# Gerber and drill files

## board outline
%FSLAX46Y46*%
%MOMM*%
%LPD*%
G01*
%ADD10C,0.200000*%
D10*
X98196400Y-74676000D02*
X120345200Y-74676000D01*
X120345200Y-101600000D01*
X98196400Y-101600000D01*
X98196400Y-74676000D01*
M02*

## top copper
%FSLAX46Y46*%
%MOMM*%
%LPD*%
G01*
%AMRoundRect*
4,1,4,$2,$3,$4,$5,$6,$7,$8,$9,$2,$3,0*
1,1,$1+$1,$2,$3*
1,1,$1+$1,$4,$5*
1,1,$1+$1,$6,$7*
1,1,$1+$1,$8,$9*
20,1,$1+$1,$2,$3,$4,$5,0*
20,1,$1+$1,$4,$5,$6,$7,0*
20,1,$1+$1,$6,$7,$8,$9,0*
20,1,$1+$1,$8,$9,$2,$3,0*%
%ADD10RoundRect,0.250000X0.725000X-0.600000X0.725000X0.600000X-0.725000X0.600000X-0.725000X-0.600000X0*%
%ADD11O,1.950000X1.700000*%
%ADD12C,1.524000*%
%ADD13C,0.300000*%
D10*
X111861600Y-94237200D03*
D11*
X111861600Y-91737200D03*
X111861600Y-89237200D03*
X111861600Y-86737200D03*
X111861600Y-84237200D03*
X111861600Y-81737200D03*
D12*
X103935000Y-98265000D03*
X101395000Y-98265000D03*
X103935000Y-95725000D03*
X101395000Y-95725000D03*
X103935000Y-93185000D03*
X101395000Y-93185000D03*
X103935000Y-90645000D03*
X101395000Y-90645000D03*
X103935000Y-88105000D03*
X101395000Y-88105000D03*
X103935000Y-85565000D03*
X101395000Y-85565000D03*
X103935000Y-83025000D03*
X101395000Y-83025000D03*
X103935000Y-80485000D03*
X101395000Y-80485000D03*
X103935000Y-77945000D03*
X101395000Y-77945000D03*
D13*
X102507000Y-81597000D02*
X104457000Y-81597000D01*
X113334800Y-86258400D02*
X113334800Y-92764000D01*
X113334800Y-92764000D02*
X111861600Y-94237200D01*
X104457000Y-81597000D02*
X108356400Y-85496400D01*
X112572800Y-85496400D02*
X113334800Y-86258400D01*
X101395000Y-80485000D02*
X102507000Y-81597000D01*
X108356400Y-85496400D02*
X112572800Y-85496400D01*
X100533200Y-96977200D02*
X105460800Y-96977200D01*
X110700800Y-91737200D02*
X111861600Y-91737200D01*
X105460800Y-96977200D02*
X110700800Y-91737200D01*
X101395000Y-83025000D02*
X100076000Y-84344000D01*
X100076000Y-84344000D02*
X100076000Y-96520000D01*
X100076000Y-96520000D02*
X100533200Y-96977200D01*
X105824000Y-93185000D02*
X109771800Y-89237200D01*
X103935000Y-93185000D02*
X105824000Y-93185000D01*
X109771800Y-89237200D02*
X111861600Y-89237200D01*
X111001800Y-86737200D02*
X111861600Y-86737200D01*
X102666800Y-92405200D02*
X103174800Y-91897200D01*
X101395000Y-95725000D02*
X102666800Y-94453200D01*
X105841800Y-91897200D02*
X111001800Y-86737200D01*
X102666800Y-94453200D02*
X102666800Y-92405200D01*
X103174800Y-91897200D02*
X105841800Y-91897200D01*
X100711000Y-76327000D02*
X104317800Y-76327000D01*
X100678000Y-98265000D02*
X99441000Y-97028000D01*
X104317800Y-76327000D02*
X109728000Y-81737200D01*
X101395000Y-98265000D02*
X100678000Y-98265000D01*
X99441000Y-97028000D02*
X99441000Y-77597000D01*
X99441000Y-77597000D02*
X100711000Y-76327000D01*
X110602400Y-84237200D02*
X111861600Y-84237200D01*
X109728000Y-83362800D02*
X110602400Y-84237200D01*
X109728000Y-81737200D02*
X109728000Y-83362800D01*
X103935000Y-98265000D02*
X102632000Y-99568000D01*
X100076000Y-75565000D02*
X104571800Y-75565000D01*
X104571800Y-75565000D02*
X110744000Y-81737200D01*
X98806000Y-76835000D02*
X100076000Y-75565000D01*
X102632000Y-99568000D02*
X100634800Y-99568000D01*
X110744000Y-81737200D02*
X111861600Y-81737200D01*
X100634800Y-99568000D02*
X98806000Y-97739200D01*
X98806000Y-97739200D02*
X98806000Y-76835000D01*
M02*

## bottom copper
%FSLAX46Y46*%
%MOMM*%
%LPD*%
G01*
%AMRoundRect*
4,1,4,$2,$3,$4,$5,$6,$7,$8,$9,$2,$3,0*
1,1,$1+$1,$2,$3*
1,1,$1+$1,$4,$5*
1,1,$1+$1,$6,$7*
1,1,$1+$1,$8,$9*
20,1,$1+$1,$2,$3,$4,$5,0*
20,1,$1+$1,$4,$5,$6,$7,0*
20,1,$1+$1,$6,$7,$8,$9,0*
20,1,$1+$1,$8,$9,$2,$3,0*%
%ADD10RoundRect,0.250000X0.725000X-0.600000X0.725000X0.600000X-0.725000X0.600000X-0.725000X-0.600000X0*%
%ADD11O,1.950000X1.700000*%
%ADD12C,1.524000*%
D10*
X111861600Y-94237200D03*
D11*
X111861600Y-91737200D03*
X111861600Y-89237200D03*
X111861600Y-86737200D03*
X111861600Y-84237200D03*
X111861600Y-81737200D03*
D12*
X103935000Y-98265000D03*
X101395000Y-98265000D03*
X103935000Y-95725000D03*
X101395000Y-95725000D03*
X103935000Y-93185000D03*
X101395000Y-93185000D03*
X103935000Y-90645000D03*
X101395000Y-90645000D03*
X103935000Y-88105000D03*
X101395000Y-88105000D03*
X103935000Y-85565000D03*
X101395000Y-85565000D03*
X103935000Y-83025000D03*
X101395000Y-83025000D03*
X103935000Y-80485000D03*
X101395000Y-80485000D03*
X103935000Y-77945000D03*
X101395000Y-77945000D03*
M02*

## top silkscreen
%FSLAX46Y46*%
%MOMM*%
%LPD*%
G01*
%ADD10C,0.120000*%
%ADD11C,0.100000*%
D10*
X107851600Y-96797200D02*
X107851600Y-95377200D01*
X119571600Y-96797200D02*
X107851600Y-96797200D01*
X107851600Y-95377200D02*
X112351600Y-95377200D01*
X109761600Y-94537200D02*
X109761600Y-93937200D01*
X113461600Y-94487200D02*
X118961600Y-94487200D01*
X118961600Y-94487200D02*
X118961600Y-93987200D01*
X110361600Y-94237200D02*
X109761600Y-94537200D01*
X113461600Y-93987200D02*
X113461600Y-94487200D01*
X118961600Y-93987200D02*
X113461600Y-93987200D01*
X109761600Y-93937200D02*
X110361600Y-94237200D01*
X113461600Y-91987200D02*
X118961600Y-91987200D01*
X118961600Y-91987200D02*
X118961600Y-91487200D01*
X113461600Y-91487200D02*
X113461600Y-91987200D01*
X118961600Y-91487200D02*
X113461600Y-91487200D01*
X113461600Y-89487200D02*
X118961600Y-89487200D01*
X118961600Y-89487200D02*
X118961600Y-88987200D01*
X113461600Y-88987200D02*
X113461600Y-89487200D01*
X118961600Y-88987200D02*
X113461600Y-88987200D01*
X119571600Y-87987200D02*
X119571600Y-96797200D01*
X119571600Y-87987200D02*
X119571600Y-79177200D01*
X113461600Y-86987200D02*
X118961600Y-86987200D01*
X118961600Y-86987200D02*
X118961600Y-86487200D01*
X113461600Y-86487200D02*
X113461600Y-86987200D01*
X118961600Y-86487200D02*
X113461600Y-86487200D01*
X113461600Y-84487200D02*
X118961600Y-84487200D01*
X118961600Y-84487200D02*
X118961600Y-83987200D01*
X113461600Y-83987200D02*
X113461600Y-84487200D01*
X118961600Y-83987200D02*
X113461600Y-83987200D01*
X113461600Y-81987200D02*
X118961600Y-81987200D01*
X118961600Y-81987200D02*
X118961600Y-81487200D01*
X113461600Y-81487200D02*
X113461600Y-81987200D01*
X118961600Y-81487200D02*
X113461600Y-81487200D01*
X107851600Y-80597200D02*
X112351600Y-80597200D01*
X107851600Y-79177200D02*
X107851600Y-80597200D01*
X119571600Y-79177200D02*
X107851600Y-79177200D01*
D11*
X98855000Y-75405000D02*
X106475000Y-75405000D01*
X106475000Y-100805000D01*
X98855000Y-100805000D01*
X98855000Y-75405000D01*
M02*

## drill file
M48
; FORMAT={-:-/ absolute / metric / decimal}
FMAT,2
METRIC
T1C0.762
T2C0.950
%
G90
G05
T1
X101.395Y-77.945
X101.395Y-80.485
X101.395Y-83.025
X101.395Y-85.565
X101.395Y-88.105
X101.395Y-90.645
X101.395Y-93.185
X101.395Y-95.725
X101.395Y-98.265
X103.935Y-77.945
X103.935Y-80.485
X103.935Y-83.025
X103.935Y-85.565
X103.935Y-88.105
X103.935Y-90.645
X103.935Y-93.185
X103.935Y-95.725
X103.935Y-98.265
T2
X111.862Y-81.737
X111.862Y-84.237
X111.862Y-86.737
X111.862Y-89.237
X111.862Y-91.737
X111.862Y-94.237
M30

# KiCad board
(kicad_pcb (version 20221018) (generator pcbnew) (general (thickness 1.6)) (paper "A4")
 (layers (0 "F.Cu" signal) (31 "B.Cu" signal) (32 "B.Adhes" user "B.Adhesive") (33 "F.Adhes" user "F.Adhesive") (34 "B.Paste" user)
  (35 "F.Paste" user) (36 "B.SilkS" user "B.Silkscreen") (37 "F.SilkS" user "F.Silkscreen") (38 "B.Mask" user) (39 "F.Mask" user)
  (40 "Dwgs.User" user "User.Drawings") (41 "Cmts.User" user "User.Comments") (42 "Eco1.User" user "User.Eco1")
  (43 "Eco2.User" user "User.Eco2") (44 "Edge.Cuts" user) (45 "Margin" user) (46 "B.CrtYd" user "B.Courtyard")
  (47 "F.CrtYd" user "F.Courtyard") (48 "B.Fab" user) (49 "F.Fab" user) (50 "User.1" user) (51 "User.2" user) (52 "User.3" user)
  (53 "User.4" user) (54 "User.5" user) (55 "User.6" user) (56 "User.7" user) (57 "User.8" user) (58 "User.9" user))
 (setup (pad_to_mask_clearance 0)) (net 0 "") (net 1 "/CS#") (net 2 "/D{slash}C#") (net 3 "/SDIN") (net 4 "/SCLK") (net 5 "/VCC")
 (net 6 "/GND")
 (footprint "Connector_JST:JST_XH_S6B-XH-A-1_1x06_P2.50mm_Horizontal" (layer "F.Cu") (at 111.8616 94.2372 90)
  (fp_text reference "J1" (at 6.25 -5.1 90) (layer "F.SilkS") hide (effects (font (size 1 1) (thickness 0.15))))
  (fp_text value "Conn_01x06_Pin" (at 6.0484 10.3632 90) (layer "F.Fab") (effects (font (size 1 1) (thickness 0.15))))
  (fp_line (start -2.56 -4.01) (end -1.14 -4.01) (stroke (width 0.12) (type solid)) (layer "F.SilkS"))
  (fp_line (start -2.56 7.71) (end -2.56 -4.01) (stroke (width 0.12) (type solid)) (layer "F.SilkS"))
  (fp_line (start -1.14 -4.01) (end -1.14 0.49) (stroke (width 0.12) (type solid)) (layer "F.SilkS"))
  (fp_line (start -0.3 -2.1) (end 0.3 -2.1) (stroke (width 0.12) (type solid)) (layer "F.SilkS"))
  (fp_line (start -0.25 1.6) (end -0.25 7.1) (stroke (width 0.12) (type solid)) (layer "F.SilkS"))
  (fp_line (start -0.25 7.1) (end 0.25 7.1) (stroke (width 0.12) (type solid)) (layer "F.SilkS"))
  (fp_line (start 0 -1.5) (end -0.3 -2.1) (stroke (width 0.12) (type solid)) (layer "F.SilkS"))
  (fp_line (start 0.25 1.6) (end -0.25 1.6) (stroke (width 0.12) (type solid)) (layer "F.SilkS"))
  (fp_line (start 0.25 7.1) (end 0.25 1.6) (stroke (width 0.12) (type solid)) (layer "F.SilkS"))
  (fp_line (start 0.3 -2.1) (end 0 -1.5) (stroke (width 0.12) (type solid)) (layer "F.SilkS"))
  (fp_line (start 2.25 1.6) (end 2.25 7.1) (stroke (width 0.12) (type solid)) (layer "F.SilkS"))
  (fp_line (start 2.25 7.1) (end 2.75 7.1) (stroke (width 0.12) (type solid)) (layer "F.SilkS"))
  (fp_line (start 2.75 1.6) (end 2.25 1.6) (stroke (width 0.12) (type solid)) (layer "F.SilkS"))
  (fp_line (start 2.75 7.1) (end 2.75 1.6) (stroke (width 0.12) (type solid)) (layer "F.SilkS"))
  (fp_line (start 4.75 1.6) (end 4.75 7.1) (stroke (width 0.12) (type solid)) (layer "F.SilkS"))
  (fp_line (start 4.75 7.1) (end 5.25 7.1) (stroke (width 0.12) (type solid)) (layer "F.SilkS"))
  (fp_line (start 5.25 1.6) (end 4.75 1.6) (stroke (width 0.12) (type solid)) (layer "F.SilkS"))
  (fp_line (start 5.25 7.1) (end 5.25 1.6) (stroke (width 0.12) (type solid)) (layer "F.SilkS"))
  (fp_line (start 6.25 7.71) (end -2.56 7.71) (stroke (width 0.12) (type solid)) (layer "F.SilkS"))
  (fp_line (start 6.25 7.71) (end 15.06 7.71) (stroke (width 0.12) (type solid)) (layer "F.SilkS"))
  (fp_line (start 7.25 1.6) (end 7.25 7.1) (stroke (width 0.12) (type solid)) (layer "F.SilkS"))
  (fp_line (start 7.25 7.1) (end 7.75 7.1) (stroke (width 0.12) (type solid)) (layer "F.SilkS"))
  (fp_line (start 7.75 1.6) (end 7.25 1.6) (stroke (width 0.12) (type solid)) (layer "F.SilkS"))
  (fp_line (start 7.75 7.1) (end 7.75 1.6) (stroke (width 0.12) (type solid)) (layer "F.SilkS"))
  (fp_line (start 9.75 1.6) (end 9.75 7.1) (stroke (width 0.12) (type solid)) (layer "F.SilkS"))
  (fp_line (start 9.75 7.1) (end 10.25 7.1) (stroke (width 0.12) (type solid)) (layer "F.SilkS"))
  (fp_line (start 10.25 1.6) (end 9.75 1.6) (stroke (width 0.12) (type solid)) (layer "F.SilkS"))
  (fp_line (start 10.25 7.1) (end 10.25 1.6) (stroke (width 0.12) (type solid)) (layer "F.SilkS"))
  (fp_line (start 12.25 1.6) (end 12.25 7.1) (stroke (width 0.12) (type solid)) (layer "F.SilkS"))
  (fp_line (start 12.25 7.1) (end 12.75 7.1) (stroke (width 0.12) (type solid)) (layer "F.SilkS"))
  (fp_line (start 12.75 1.6) (end 12.25 1.6) (stroke (width 0.12) (type solid)) (layer "F.SilkS"))
  (fp_line (start 12.75 7.1) (end 12.75 1.6) (stroke (width 0.12) (type solid)) (layer "F.SilkS"))
  (fp_line (start 13.64 -4.01) (end 13.64 0.49) (stroke (width 0.12) (type solid)) (layer "F.SilkS"))
  (fp_line (start 15.06 -4.01) (end 13.64 -4.01) (stroke (width 0.12) (type solid)) (layer "F.SilkS"))
  (fp_line (start 15.06 7.71) (end 15.06 -4.01) (stroke (width 0.12) (type solid)) (layer "F.SilkS"))
  (pad "1" thru_hole roundrect (at 0 0 90) (size 1.7 1.95) (drill 0.95) (layers "*.Cu" "*.Mask") (roundrect_rratio 0.147059) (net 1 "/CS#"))
  (pad "2" thru_hole oval (at 2.5 0 90) (size 1.7 1.95) (drill 0.95) (layers "*.Cu" "*.Mask") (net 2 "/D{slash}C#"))
  (pad "3" thru_hole oval (at 5 0 90) (size 1.7 1.95) (drill 0.95) (layers "*.Cu" "*.Mask") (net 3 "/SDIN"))
  (pad "4" thru_hole oval (at 7.5 0 90) (size 1.7 1.95) (drill 0.95) (layers "*.Cu" "*.Mask") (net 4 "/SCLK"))
  (pad "5" thru_hole oval (at 10 0 90) (size 1.7 1.95) (drill 0.95) (layers "*.Cu" "*.Mask") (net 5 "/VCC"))
  (pad "6" thru_hole oval (at 12.5 0 90) (size 1.7 1.95) (drill 0.95) (layers "*.Cu" "*.Mask") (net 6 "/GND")))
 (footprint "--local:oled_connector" (layer "F.Cu") (at 101.395 70.325)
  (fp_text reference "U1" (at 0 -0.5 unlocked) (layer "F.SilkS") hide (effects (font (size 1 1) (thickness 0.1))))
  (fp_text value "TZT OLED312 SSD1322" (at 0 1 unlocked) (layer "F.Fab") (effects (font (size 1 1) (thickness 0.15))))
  (fp_rect (start -2.54 5.08) (end 5.08 30.48) (stroke (width 0.1) (type default)) (fill none) (layer "F.SilkS"))
  (pad "1" thru_hole circle (at 2.54 27.94) (size 1.524 1.524) (drill 0.762) (layers "*.Cu" "*.Mask") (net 6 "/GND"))
  (pad "2" thru_hole circle (at 0 27.94) (size 1.524 1.524) (drill 0.762) (layers "*.Cu" "*.Mask") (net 5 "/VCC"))
  (pad "3" thru_hole circle (at 2.54 25.4) (size 1.524 1.524) (drill 0.762) (layers "*.Cu" "*.Mask"))
  (pad "4" thru_hole circle (at 0 25.4) (size 1.524 1.524) (drill 0.762) (layers "*.Cu" "*.Mask") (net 4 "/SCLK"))
  (pad "5" thru_hole circle (at 2.54 22.86) (size 1.524 1.524) (drill 0.762) (layers "*.Cu" "*.Mask") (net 3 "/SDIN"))
  (pad "6" thru_hole circle (at 0 22.86) (size 1.524 1.524) (drill 0.762) (layers "*.Cu" "*.Mask"))
  (pad "7" thru_hole circle (at 2.54 20.32) (size 1.524 1.524) (drill 0.762) (layers "*.Cu" "*.Mask"))
  (pad "8" thru_hole circle (at 0 20.32) (size 1.524 1.524) (drill 0.762) (layers "*.Cu" "*.Mask"))
  (pad "9" thru_hole circle (at 2.54 17.78) (size 1.524 1.524) (drill 0.762) (layers "*.Cu" "*.Mask"))
  (pad "10" thru_hole circle (at 0 17.78) (size 1.524 1.524) (drill 0.762) (layers "*.Cu" "*.Mask"))
  (pad "11" thru_hole circle (at 2.54 15.24) (size 1.524 1.524) (drill 0.762) (layers "*.Cu" "*.Mask"))
  (pad "12" thru_hole circle (at 0 15.24) (size 1.524 1.524) (drill 0.762) (layers "*.Cu" "*.Mask"))
  (pad "13" thru_hole circle (at 2.54 12.7) (size 1.524 1.524) (drill 0.762) (layers "*.Cu" "*.Mask"))
  (pad "14" thru_hole circle (at 0 12.7) (size 1.524 1.524) (drill 0.762) (layers "*.Cu" "*.Mask") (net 2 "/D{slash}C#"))
  (pad "15" thru_hole circle (at 2.54 10.16) (size 1.524 1.524) (drill 0.762) (layers "*.Cu" "*.Mask"))
  (pad "16" thru_hole circle (at 0 10.16) (size 1.524 1.524) (drill 0.762) (layers "*.Cu" "*.Mask") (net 1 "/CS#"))
  (pad "17" thru_hole circle (at 2.54 7.62) (size 1.524 1.524) (drill 0.762) (layers "*.Cu" "*.Mask"))
  (pad "18" thru_hole circle (at 0 7.62) (size 1.524 1.524) (drill 0.762) (layers "*.Cu" "*.Mask")))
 (gr_rect (start 98.1964 74.676) (end 120.3452 101.6) (stroke (width 0.2) (type default)) (fill none) (layer "Edge.Cuts"))
 (segment (start 102.507 81.597) (end 104.457 81.597) (width 0.3) (layer "F.Cu") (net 1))
 (segment (start 113.3348 86.2584) (end 113.3348 92.764) (width 0.3) (layer "F.Cu") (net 1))
 (segment (start 113.3348 92.764) (end 111.8616 94.2372) (width 0.3) (layer "F.Cu") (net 1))
 (segment (start 104.457 81.597) (end 108.3564 85.4964) (width 0.3) (layer "F.Cu") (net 1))
 (segment (start 112.5728 85.4964) (end 113.3348 86.2584) (width 0.3) (layer "F.Cu") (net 1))
 (segment (start 101.395 80.485) (end 102.507 81.597) (width 0.3) (layer "F.Cu") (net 1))
 (segment (start 108.3564 85.4964) (end 112.5728 85.4964) (width 0.3) (layer "F.Cu") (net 1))
 (segment (start 100.5332 96.9772) (end 105.4608 96.9772) (width 0.3) (layer "F.Cu") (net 2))
 (segment (start 110.7008 91.7372) (end 111.8616 91.7372) (width 0.3) (layer "F.Cu") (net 2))
 (segment (start 105.4608 96.9772) (end 110.7008 91.7372) (width 0.3) (layer "F.Cu") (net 2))
 (segment (start 101.395 83.025) (end 100.076 84.344) (width 0.3) (layer "F.Cu") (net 2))
 (segment (start 100.076 84.344) (end 100.076 96.52) (width 0.3) (layer "F.Cu") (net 2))
 (segment (start 100.076 96.52) (end 100.5332 96.9772) (width 0.3) (layer "F.Cu") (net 2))
 (segment (start 105.824 93.185) (end 109.7718 89.2372) (width 0.3) (layer "F.Cu") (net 3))
 (segment (start 103.935 93.185) (end 105.824 93.185) (width 0.3) (layer "F.Cu") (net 3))
 (segment (start 109.7718 89.2372) (end 111.8616 89.2372) (width 0.3) (layer "F.Cu") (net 3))
 (segment (start 111.0018 86.7372) (end 111.8616 86.7372) (width 0.3) (layer "F.Cu") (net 4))
 (segment (start 102.6668 92.4052) (end 103.1748 91.8972) (width 0.3) (layer "F.Cu") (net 4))
 (segment (start 101.395 95.725) (end 102.6668 94.4532) (width 0.3) (layer "F.Cu") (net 4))
 (segment (start 105.8418 91.8972) (end 111.0018 86.7372) (width 0.3) (layer "F.Cu") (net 4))
 (segment (start 102.6668 94.4532) (end 102.6668 92.4052) (width 0.3) (layer "F.Cu") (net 4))
 (segment (start 103.1748 91.8972) (end 105.8418 91.8972) (width 0.3) (layer "F.Cu") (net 4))
 (segment (start 100.711 76.327) (end 104.3178 76.327) (width 0.3) (layer "F.Cu") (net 5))
 (segment (start 100.678 98.265) (end 99.441 97.028) (width 0.3) (layer "F.Cu") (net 5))
 (segment (start 104.3178 76.327) (end 109.728 81.7372) (width 0.3) (layer "F.Cu") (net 5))
 (segment (start 101.395 98.265) (end 100.678 98.265) (width 0.3) (layer "F.Cu") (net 5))
 (segment (start 99.441 97.028) (end 99.441 77.597) (width 0.3) (layer "F.Cu") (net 5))
 (segment (start 99.441 77.597) (end 100.711 76.327) (width 0.3) (layer "F.Cu") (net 5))
 (segment (start 110.6024 84.2372) (end 111.8616 84.2372) (width 0.3) (layer "F.Cu") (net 5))
 (segment (start 109.728 83.3628) (end 110.6024 84.2372) (width 0.3) (layer "F.Cu") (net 5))
 (segment (start 109.728 81.7372) (end 109.728 83.3628) (width 0.3) (layer "F.Cu") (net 5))
 (segment (start 103.935 98.265) (end 102.632 99.568) (width 0.3) (layer "F.Cu") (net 6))
 (segment (start 100.076 75.565) (end 104.5718 75.565) (width 0.3) (layer "F.Cu") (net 6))
 (segment (start 104.5718 75.565) (end 110.744 81.7372) (width 0.3) (layer "F.Cu") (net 6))
 (segment (start 98.806 76.835) (end 100.076 75.565) (width 0.3) (layer "F.Cu") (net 6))
 (segment (start 102.632 99.568) (end 100.6348 99.568) (width 0.3) (layer "F.Cu") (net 6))
 (segment (start 110.744 81.7372) (end 111.8616 81.7372) (width 0.3) (layer "F.Cu") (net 6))
 (segment (start 100.6348 99.568) (end 98.806 97.7392) (width 0.3) (layer "F.Cu") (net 6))
 (segment (start 98.806 97.7392) (end 98.806 76.835) (width 0.3) (layer "F.Cu") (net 6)))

